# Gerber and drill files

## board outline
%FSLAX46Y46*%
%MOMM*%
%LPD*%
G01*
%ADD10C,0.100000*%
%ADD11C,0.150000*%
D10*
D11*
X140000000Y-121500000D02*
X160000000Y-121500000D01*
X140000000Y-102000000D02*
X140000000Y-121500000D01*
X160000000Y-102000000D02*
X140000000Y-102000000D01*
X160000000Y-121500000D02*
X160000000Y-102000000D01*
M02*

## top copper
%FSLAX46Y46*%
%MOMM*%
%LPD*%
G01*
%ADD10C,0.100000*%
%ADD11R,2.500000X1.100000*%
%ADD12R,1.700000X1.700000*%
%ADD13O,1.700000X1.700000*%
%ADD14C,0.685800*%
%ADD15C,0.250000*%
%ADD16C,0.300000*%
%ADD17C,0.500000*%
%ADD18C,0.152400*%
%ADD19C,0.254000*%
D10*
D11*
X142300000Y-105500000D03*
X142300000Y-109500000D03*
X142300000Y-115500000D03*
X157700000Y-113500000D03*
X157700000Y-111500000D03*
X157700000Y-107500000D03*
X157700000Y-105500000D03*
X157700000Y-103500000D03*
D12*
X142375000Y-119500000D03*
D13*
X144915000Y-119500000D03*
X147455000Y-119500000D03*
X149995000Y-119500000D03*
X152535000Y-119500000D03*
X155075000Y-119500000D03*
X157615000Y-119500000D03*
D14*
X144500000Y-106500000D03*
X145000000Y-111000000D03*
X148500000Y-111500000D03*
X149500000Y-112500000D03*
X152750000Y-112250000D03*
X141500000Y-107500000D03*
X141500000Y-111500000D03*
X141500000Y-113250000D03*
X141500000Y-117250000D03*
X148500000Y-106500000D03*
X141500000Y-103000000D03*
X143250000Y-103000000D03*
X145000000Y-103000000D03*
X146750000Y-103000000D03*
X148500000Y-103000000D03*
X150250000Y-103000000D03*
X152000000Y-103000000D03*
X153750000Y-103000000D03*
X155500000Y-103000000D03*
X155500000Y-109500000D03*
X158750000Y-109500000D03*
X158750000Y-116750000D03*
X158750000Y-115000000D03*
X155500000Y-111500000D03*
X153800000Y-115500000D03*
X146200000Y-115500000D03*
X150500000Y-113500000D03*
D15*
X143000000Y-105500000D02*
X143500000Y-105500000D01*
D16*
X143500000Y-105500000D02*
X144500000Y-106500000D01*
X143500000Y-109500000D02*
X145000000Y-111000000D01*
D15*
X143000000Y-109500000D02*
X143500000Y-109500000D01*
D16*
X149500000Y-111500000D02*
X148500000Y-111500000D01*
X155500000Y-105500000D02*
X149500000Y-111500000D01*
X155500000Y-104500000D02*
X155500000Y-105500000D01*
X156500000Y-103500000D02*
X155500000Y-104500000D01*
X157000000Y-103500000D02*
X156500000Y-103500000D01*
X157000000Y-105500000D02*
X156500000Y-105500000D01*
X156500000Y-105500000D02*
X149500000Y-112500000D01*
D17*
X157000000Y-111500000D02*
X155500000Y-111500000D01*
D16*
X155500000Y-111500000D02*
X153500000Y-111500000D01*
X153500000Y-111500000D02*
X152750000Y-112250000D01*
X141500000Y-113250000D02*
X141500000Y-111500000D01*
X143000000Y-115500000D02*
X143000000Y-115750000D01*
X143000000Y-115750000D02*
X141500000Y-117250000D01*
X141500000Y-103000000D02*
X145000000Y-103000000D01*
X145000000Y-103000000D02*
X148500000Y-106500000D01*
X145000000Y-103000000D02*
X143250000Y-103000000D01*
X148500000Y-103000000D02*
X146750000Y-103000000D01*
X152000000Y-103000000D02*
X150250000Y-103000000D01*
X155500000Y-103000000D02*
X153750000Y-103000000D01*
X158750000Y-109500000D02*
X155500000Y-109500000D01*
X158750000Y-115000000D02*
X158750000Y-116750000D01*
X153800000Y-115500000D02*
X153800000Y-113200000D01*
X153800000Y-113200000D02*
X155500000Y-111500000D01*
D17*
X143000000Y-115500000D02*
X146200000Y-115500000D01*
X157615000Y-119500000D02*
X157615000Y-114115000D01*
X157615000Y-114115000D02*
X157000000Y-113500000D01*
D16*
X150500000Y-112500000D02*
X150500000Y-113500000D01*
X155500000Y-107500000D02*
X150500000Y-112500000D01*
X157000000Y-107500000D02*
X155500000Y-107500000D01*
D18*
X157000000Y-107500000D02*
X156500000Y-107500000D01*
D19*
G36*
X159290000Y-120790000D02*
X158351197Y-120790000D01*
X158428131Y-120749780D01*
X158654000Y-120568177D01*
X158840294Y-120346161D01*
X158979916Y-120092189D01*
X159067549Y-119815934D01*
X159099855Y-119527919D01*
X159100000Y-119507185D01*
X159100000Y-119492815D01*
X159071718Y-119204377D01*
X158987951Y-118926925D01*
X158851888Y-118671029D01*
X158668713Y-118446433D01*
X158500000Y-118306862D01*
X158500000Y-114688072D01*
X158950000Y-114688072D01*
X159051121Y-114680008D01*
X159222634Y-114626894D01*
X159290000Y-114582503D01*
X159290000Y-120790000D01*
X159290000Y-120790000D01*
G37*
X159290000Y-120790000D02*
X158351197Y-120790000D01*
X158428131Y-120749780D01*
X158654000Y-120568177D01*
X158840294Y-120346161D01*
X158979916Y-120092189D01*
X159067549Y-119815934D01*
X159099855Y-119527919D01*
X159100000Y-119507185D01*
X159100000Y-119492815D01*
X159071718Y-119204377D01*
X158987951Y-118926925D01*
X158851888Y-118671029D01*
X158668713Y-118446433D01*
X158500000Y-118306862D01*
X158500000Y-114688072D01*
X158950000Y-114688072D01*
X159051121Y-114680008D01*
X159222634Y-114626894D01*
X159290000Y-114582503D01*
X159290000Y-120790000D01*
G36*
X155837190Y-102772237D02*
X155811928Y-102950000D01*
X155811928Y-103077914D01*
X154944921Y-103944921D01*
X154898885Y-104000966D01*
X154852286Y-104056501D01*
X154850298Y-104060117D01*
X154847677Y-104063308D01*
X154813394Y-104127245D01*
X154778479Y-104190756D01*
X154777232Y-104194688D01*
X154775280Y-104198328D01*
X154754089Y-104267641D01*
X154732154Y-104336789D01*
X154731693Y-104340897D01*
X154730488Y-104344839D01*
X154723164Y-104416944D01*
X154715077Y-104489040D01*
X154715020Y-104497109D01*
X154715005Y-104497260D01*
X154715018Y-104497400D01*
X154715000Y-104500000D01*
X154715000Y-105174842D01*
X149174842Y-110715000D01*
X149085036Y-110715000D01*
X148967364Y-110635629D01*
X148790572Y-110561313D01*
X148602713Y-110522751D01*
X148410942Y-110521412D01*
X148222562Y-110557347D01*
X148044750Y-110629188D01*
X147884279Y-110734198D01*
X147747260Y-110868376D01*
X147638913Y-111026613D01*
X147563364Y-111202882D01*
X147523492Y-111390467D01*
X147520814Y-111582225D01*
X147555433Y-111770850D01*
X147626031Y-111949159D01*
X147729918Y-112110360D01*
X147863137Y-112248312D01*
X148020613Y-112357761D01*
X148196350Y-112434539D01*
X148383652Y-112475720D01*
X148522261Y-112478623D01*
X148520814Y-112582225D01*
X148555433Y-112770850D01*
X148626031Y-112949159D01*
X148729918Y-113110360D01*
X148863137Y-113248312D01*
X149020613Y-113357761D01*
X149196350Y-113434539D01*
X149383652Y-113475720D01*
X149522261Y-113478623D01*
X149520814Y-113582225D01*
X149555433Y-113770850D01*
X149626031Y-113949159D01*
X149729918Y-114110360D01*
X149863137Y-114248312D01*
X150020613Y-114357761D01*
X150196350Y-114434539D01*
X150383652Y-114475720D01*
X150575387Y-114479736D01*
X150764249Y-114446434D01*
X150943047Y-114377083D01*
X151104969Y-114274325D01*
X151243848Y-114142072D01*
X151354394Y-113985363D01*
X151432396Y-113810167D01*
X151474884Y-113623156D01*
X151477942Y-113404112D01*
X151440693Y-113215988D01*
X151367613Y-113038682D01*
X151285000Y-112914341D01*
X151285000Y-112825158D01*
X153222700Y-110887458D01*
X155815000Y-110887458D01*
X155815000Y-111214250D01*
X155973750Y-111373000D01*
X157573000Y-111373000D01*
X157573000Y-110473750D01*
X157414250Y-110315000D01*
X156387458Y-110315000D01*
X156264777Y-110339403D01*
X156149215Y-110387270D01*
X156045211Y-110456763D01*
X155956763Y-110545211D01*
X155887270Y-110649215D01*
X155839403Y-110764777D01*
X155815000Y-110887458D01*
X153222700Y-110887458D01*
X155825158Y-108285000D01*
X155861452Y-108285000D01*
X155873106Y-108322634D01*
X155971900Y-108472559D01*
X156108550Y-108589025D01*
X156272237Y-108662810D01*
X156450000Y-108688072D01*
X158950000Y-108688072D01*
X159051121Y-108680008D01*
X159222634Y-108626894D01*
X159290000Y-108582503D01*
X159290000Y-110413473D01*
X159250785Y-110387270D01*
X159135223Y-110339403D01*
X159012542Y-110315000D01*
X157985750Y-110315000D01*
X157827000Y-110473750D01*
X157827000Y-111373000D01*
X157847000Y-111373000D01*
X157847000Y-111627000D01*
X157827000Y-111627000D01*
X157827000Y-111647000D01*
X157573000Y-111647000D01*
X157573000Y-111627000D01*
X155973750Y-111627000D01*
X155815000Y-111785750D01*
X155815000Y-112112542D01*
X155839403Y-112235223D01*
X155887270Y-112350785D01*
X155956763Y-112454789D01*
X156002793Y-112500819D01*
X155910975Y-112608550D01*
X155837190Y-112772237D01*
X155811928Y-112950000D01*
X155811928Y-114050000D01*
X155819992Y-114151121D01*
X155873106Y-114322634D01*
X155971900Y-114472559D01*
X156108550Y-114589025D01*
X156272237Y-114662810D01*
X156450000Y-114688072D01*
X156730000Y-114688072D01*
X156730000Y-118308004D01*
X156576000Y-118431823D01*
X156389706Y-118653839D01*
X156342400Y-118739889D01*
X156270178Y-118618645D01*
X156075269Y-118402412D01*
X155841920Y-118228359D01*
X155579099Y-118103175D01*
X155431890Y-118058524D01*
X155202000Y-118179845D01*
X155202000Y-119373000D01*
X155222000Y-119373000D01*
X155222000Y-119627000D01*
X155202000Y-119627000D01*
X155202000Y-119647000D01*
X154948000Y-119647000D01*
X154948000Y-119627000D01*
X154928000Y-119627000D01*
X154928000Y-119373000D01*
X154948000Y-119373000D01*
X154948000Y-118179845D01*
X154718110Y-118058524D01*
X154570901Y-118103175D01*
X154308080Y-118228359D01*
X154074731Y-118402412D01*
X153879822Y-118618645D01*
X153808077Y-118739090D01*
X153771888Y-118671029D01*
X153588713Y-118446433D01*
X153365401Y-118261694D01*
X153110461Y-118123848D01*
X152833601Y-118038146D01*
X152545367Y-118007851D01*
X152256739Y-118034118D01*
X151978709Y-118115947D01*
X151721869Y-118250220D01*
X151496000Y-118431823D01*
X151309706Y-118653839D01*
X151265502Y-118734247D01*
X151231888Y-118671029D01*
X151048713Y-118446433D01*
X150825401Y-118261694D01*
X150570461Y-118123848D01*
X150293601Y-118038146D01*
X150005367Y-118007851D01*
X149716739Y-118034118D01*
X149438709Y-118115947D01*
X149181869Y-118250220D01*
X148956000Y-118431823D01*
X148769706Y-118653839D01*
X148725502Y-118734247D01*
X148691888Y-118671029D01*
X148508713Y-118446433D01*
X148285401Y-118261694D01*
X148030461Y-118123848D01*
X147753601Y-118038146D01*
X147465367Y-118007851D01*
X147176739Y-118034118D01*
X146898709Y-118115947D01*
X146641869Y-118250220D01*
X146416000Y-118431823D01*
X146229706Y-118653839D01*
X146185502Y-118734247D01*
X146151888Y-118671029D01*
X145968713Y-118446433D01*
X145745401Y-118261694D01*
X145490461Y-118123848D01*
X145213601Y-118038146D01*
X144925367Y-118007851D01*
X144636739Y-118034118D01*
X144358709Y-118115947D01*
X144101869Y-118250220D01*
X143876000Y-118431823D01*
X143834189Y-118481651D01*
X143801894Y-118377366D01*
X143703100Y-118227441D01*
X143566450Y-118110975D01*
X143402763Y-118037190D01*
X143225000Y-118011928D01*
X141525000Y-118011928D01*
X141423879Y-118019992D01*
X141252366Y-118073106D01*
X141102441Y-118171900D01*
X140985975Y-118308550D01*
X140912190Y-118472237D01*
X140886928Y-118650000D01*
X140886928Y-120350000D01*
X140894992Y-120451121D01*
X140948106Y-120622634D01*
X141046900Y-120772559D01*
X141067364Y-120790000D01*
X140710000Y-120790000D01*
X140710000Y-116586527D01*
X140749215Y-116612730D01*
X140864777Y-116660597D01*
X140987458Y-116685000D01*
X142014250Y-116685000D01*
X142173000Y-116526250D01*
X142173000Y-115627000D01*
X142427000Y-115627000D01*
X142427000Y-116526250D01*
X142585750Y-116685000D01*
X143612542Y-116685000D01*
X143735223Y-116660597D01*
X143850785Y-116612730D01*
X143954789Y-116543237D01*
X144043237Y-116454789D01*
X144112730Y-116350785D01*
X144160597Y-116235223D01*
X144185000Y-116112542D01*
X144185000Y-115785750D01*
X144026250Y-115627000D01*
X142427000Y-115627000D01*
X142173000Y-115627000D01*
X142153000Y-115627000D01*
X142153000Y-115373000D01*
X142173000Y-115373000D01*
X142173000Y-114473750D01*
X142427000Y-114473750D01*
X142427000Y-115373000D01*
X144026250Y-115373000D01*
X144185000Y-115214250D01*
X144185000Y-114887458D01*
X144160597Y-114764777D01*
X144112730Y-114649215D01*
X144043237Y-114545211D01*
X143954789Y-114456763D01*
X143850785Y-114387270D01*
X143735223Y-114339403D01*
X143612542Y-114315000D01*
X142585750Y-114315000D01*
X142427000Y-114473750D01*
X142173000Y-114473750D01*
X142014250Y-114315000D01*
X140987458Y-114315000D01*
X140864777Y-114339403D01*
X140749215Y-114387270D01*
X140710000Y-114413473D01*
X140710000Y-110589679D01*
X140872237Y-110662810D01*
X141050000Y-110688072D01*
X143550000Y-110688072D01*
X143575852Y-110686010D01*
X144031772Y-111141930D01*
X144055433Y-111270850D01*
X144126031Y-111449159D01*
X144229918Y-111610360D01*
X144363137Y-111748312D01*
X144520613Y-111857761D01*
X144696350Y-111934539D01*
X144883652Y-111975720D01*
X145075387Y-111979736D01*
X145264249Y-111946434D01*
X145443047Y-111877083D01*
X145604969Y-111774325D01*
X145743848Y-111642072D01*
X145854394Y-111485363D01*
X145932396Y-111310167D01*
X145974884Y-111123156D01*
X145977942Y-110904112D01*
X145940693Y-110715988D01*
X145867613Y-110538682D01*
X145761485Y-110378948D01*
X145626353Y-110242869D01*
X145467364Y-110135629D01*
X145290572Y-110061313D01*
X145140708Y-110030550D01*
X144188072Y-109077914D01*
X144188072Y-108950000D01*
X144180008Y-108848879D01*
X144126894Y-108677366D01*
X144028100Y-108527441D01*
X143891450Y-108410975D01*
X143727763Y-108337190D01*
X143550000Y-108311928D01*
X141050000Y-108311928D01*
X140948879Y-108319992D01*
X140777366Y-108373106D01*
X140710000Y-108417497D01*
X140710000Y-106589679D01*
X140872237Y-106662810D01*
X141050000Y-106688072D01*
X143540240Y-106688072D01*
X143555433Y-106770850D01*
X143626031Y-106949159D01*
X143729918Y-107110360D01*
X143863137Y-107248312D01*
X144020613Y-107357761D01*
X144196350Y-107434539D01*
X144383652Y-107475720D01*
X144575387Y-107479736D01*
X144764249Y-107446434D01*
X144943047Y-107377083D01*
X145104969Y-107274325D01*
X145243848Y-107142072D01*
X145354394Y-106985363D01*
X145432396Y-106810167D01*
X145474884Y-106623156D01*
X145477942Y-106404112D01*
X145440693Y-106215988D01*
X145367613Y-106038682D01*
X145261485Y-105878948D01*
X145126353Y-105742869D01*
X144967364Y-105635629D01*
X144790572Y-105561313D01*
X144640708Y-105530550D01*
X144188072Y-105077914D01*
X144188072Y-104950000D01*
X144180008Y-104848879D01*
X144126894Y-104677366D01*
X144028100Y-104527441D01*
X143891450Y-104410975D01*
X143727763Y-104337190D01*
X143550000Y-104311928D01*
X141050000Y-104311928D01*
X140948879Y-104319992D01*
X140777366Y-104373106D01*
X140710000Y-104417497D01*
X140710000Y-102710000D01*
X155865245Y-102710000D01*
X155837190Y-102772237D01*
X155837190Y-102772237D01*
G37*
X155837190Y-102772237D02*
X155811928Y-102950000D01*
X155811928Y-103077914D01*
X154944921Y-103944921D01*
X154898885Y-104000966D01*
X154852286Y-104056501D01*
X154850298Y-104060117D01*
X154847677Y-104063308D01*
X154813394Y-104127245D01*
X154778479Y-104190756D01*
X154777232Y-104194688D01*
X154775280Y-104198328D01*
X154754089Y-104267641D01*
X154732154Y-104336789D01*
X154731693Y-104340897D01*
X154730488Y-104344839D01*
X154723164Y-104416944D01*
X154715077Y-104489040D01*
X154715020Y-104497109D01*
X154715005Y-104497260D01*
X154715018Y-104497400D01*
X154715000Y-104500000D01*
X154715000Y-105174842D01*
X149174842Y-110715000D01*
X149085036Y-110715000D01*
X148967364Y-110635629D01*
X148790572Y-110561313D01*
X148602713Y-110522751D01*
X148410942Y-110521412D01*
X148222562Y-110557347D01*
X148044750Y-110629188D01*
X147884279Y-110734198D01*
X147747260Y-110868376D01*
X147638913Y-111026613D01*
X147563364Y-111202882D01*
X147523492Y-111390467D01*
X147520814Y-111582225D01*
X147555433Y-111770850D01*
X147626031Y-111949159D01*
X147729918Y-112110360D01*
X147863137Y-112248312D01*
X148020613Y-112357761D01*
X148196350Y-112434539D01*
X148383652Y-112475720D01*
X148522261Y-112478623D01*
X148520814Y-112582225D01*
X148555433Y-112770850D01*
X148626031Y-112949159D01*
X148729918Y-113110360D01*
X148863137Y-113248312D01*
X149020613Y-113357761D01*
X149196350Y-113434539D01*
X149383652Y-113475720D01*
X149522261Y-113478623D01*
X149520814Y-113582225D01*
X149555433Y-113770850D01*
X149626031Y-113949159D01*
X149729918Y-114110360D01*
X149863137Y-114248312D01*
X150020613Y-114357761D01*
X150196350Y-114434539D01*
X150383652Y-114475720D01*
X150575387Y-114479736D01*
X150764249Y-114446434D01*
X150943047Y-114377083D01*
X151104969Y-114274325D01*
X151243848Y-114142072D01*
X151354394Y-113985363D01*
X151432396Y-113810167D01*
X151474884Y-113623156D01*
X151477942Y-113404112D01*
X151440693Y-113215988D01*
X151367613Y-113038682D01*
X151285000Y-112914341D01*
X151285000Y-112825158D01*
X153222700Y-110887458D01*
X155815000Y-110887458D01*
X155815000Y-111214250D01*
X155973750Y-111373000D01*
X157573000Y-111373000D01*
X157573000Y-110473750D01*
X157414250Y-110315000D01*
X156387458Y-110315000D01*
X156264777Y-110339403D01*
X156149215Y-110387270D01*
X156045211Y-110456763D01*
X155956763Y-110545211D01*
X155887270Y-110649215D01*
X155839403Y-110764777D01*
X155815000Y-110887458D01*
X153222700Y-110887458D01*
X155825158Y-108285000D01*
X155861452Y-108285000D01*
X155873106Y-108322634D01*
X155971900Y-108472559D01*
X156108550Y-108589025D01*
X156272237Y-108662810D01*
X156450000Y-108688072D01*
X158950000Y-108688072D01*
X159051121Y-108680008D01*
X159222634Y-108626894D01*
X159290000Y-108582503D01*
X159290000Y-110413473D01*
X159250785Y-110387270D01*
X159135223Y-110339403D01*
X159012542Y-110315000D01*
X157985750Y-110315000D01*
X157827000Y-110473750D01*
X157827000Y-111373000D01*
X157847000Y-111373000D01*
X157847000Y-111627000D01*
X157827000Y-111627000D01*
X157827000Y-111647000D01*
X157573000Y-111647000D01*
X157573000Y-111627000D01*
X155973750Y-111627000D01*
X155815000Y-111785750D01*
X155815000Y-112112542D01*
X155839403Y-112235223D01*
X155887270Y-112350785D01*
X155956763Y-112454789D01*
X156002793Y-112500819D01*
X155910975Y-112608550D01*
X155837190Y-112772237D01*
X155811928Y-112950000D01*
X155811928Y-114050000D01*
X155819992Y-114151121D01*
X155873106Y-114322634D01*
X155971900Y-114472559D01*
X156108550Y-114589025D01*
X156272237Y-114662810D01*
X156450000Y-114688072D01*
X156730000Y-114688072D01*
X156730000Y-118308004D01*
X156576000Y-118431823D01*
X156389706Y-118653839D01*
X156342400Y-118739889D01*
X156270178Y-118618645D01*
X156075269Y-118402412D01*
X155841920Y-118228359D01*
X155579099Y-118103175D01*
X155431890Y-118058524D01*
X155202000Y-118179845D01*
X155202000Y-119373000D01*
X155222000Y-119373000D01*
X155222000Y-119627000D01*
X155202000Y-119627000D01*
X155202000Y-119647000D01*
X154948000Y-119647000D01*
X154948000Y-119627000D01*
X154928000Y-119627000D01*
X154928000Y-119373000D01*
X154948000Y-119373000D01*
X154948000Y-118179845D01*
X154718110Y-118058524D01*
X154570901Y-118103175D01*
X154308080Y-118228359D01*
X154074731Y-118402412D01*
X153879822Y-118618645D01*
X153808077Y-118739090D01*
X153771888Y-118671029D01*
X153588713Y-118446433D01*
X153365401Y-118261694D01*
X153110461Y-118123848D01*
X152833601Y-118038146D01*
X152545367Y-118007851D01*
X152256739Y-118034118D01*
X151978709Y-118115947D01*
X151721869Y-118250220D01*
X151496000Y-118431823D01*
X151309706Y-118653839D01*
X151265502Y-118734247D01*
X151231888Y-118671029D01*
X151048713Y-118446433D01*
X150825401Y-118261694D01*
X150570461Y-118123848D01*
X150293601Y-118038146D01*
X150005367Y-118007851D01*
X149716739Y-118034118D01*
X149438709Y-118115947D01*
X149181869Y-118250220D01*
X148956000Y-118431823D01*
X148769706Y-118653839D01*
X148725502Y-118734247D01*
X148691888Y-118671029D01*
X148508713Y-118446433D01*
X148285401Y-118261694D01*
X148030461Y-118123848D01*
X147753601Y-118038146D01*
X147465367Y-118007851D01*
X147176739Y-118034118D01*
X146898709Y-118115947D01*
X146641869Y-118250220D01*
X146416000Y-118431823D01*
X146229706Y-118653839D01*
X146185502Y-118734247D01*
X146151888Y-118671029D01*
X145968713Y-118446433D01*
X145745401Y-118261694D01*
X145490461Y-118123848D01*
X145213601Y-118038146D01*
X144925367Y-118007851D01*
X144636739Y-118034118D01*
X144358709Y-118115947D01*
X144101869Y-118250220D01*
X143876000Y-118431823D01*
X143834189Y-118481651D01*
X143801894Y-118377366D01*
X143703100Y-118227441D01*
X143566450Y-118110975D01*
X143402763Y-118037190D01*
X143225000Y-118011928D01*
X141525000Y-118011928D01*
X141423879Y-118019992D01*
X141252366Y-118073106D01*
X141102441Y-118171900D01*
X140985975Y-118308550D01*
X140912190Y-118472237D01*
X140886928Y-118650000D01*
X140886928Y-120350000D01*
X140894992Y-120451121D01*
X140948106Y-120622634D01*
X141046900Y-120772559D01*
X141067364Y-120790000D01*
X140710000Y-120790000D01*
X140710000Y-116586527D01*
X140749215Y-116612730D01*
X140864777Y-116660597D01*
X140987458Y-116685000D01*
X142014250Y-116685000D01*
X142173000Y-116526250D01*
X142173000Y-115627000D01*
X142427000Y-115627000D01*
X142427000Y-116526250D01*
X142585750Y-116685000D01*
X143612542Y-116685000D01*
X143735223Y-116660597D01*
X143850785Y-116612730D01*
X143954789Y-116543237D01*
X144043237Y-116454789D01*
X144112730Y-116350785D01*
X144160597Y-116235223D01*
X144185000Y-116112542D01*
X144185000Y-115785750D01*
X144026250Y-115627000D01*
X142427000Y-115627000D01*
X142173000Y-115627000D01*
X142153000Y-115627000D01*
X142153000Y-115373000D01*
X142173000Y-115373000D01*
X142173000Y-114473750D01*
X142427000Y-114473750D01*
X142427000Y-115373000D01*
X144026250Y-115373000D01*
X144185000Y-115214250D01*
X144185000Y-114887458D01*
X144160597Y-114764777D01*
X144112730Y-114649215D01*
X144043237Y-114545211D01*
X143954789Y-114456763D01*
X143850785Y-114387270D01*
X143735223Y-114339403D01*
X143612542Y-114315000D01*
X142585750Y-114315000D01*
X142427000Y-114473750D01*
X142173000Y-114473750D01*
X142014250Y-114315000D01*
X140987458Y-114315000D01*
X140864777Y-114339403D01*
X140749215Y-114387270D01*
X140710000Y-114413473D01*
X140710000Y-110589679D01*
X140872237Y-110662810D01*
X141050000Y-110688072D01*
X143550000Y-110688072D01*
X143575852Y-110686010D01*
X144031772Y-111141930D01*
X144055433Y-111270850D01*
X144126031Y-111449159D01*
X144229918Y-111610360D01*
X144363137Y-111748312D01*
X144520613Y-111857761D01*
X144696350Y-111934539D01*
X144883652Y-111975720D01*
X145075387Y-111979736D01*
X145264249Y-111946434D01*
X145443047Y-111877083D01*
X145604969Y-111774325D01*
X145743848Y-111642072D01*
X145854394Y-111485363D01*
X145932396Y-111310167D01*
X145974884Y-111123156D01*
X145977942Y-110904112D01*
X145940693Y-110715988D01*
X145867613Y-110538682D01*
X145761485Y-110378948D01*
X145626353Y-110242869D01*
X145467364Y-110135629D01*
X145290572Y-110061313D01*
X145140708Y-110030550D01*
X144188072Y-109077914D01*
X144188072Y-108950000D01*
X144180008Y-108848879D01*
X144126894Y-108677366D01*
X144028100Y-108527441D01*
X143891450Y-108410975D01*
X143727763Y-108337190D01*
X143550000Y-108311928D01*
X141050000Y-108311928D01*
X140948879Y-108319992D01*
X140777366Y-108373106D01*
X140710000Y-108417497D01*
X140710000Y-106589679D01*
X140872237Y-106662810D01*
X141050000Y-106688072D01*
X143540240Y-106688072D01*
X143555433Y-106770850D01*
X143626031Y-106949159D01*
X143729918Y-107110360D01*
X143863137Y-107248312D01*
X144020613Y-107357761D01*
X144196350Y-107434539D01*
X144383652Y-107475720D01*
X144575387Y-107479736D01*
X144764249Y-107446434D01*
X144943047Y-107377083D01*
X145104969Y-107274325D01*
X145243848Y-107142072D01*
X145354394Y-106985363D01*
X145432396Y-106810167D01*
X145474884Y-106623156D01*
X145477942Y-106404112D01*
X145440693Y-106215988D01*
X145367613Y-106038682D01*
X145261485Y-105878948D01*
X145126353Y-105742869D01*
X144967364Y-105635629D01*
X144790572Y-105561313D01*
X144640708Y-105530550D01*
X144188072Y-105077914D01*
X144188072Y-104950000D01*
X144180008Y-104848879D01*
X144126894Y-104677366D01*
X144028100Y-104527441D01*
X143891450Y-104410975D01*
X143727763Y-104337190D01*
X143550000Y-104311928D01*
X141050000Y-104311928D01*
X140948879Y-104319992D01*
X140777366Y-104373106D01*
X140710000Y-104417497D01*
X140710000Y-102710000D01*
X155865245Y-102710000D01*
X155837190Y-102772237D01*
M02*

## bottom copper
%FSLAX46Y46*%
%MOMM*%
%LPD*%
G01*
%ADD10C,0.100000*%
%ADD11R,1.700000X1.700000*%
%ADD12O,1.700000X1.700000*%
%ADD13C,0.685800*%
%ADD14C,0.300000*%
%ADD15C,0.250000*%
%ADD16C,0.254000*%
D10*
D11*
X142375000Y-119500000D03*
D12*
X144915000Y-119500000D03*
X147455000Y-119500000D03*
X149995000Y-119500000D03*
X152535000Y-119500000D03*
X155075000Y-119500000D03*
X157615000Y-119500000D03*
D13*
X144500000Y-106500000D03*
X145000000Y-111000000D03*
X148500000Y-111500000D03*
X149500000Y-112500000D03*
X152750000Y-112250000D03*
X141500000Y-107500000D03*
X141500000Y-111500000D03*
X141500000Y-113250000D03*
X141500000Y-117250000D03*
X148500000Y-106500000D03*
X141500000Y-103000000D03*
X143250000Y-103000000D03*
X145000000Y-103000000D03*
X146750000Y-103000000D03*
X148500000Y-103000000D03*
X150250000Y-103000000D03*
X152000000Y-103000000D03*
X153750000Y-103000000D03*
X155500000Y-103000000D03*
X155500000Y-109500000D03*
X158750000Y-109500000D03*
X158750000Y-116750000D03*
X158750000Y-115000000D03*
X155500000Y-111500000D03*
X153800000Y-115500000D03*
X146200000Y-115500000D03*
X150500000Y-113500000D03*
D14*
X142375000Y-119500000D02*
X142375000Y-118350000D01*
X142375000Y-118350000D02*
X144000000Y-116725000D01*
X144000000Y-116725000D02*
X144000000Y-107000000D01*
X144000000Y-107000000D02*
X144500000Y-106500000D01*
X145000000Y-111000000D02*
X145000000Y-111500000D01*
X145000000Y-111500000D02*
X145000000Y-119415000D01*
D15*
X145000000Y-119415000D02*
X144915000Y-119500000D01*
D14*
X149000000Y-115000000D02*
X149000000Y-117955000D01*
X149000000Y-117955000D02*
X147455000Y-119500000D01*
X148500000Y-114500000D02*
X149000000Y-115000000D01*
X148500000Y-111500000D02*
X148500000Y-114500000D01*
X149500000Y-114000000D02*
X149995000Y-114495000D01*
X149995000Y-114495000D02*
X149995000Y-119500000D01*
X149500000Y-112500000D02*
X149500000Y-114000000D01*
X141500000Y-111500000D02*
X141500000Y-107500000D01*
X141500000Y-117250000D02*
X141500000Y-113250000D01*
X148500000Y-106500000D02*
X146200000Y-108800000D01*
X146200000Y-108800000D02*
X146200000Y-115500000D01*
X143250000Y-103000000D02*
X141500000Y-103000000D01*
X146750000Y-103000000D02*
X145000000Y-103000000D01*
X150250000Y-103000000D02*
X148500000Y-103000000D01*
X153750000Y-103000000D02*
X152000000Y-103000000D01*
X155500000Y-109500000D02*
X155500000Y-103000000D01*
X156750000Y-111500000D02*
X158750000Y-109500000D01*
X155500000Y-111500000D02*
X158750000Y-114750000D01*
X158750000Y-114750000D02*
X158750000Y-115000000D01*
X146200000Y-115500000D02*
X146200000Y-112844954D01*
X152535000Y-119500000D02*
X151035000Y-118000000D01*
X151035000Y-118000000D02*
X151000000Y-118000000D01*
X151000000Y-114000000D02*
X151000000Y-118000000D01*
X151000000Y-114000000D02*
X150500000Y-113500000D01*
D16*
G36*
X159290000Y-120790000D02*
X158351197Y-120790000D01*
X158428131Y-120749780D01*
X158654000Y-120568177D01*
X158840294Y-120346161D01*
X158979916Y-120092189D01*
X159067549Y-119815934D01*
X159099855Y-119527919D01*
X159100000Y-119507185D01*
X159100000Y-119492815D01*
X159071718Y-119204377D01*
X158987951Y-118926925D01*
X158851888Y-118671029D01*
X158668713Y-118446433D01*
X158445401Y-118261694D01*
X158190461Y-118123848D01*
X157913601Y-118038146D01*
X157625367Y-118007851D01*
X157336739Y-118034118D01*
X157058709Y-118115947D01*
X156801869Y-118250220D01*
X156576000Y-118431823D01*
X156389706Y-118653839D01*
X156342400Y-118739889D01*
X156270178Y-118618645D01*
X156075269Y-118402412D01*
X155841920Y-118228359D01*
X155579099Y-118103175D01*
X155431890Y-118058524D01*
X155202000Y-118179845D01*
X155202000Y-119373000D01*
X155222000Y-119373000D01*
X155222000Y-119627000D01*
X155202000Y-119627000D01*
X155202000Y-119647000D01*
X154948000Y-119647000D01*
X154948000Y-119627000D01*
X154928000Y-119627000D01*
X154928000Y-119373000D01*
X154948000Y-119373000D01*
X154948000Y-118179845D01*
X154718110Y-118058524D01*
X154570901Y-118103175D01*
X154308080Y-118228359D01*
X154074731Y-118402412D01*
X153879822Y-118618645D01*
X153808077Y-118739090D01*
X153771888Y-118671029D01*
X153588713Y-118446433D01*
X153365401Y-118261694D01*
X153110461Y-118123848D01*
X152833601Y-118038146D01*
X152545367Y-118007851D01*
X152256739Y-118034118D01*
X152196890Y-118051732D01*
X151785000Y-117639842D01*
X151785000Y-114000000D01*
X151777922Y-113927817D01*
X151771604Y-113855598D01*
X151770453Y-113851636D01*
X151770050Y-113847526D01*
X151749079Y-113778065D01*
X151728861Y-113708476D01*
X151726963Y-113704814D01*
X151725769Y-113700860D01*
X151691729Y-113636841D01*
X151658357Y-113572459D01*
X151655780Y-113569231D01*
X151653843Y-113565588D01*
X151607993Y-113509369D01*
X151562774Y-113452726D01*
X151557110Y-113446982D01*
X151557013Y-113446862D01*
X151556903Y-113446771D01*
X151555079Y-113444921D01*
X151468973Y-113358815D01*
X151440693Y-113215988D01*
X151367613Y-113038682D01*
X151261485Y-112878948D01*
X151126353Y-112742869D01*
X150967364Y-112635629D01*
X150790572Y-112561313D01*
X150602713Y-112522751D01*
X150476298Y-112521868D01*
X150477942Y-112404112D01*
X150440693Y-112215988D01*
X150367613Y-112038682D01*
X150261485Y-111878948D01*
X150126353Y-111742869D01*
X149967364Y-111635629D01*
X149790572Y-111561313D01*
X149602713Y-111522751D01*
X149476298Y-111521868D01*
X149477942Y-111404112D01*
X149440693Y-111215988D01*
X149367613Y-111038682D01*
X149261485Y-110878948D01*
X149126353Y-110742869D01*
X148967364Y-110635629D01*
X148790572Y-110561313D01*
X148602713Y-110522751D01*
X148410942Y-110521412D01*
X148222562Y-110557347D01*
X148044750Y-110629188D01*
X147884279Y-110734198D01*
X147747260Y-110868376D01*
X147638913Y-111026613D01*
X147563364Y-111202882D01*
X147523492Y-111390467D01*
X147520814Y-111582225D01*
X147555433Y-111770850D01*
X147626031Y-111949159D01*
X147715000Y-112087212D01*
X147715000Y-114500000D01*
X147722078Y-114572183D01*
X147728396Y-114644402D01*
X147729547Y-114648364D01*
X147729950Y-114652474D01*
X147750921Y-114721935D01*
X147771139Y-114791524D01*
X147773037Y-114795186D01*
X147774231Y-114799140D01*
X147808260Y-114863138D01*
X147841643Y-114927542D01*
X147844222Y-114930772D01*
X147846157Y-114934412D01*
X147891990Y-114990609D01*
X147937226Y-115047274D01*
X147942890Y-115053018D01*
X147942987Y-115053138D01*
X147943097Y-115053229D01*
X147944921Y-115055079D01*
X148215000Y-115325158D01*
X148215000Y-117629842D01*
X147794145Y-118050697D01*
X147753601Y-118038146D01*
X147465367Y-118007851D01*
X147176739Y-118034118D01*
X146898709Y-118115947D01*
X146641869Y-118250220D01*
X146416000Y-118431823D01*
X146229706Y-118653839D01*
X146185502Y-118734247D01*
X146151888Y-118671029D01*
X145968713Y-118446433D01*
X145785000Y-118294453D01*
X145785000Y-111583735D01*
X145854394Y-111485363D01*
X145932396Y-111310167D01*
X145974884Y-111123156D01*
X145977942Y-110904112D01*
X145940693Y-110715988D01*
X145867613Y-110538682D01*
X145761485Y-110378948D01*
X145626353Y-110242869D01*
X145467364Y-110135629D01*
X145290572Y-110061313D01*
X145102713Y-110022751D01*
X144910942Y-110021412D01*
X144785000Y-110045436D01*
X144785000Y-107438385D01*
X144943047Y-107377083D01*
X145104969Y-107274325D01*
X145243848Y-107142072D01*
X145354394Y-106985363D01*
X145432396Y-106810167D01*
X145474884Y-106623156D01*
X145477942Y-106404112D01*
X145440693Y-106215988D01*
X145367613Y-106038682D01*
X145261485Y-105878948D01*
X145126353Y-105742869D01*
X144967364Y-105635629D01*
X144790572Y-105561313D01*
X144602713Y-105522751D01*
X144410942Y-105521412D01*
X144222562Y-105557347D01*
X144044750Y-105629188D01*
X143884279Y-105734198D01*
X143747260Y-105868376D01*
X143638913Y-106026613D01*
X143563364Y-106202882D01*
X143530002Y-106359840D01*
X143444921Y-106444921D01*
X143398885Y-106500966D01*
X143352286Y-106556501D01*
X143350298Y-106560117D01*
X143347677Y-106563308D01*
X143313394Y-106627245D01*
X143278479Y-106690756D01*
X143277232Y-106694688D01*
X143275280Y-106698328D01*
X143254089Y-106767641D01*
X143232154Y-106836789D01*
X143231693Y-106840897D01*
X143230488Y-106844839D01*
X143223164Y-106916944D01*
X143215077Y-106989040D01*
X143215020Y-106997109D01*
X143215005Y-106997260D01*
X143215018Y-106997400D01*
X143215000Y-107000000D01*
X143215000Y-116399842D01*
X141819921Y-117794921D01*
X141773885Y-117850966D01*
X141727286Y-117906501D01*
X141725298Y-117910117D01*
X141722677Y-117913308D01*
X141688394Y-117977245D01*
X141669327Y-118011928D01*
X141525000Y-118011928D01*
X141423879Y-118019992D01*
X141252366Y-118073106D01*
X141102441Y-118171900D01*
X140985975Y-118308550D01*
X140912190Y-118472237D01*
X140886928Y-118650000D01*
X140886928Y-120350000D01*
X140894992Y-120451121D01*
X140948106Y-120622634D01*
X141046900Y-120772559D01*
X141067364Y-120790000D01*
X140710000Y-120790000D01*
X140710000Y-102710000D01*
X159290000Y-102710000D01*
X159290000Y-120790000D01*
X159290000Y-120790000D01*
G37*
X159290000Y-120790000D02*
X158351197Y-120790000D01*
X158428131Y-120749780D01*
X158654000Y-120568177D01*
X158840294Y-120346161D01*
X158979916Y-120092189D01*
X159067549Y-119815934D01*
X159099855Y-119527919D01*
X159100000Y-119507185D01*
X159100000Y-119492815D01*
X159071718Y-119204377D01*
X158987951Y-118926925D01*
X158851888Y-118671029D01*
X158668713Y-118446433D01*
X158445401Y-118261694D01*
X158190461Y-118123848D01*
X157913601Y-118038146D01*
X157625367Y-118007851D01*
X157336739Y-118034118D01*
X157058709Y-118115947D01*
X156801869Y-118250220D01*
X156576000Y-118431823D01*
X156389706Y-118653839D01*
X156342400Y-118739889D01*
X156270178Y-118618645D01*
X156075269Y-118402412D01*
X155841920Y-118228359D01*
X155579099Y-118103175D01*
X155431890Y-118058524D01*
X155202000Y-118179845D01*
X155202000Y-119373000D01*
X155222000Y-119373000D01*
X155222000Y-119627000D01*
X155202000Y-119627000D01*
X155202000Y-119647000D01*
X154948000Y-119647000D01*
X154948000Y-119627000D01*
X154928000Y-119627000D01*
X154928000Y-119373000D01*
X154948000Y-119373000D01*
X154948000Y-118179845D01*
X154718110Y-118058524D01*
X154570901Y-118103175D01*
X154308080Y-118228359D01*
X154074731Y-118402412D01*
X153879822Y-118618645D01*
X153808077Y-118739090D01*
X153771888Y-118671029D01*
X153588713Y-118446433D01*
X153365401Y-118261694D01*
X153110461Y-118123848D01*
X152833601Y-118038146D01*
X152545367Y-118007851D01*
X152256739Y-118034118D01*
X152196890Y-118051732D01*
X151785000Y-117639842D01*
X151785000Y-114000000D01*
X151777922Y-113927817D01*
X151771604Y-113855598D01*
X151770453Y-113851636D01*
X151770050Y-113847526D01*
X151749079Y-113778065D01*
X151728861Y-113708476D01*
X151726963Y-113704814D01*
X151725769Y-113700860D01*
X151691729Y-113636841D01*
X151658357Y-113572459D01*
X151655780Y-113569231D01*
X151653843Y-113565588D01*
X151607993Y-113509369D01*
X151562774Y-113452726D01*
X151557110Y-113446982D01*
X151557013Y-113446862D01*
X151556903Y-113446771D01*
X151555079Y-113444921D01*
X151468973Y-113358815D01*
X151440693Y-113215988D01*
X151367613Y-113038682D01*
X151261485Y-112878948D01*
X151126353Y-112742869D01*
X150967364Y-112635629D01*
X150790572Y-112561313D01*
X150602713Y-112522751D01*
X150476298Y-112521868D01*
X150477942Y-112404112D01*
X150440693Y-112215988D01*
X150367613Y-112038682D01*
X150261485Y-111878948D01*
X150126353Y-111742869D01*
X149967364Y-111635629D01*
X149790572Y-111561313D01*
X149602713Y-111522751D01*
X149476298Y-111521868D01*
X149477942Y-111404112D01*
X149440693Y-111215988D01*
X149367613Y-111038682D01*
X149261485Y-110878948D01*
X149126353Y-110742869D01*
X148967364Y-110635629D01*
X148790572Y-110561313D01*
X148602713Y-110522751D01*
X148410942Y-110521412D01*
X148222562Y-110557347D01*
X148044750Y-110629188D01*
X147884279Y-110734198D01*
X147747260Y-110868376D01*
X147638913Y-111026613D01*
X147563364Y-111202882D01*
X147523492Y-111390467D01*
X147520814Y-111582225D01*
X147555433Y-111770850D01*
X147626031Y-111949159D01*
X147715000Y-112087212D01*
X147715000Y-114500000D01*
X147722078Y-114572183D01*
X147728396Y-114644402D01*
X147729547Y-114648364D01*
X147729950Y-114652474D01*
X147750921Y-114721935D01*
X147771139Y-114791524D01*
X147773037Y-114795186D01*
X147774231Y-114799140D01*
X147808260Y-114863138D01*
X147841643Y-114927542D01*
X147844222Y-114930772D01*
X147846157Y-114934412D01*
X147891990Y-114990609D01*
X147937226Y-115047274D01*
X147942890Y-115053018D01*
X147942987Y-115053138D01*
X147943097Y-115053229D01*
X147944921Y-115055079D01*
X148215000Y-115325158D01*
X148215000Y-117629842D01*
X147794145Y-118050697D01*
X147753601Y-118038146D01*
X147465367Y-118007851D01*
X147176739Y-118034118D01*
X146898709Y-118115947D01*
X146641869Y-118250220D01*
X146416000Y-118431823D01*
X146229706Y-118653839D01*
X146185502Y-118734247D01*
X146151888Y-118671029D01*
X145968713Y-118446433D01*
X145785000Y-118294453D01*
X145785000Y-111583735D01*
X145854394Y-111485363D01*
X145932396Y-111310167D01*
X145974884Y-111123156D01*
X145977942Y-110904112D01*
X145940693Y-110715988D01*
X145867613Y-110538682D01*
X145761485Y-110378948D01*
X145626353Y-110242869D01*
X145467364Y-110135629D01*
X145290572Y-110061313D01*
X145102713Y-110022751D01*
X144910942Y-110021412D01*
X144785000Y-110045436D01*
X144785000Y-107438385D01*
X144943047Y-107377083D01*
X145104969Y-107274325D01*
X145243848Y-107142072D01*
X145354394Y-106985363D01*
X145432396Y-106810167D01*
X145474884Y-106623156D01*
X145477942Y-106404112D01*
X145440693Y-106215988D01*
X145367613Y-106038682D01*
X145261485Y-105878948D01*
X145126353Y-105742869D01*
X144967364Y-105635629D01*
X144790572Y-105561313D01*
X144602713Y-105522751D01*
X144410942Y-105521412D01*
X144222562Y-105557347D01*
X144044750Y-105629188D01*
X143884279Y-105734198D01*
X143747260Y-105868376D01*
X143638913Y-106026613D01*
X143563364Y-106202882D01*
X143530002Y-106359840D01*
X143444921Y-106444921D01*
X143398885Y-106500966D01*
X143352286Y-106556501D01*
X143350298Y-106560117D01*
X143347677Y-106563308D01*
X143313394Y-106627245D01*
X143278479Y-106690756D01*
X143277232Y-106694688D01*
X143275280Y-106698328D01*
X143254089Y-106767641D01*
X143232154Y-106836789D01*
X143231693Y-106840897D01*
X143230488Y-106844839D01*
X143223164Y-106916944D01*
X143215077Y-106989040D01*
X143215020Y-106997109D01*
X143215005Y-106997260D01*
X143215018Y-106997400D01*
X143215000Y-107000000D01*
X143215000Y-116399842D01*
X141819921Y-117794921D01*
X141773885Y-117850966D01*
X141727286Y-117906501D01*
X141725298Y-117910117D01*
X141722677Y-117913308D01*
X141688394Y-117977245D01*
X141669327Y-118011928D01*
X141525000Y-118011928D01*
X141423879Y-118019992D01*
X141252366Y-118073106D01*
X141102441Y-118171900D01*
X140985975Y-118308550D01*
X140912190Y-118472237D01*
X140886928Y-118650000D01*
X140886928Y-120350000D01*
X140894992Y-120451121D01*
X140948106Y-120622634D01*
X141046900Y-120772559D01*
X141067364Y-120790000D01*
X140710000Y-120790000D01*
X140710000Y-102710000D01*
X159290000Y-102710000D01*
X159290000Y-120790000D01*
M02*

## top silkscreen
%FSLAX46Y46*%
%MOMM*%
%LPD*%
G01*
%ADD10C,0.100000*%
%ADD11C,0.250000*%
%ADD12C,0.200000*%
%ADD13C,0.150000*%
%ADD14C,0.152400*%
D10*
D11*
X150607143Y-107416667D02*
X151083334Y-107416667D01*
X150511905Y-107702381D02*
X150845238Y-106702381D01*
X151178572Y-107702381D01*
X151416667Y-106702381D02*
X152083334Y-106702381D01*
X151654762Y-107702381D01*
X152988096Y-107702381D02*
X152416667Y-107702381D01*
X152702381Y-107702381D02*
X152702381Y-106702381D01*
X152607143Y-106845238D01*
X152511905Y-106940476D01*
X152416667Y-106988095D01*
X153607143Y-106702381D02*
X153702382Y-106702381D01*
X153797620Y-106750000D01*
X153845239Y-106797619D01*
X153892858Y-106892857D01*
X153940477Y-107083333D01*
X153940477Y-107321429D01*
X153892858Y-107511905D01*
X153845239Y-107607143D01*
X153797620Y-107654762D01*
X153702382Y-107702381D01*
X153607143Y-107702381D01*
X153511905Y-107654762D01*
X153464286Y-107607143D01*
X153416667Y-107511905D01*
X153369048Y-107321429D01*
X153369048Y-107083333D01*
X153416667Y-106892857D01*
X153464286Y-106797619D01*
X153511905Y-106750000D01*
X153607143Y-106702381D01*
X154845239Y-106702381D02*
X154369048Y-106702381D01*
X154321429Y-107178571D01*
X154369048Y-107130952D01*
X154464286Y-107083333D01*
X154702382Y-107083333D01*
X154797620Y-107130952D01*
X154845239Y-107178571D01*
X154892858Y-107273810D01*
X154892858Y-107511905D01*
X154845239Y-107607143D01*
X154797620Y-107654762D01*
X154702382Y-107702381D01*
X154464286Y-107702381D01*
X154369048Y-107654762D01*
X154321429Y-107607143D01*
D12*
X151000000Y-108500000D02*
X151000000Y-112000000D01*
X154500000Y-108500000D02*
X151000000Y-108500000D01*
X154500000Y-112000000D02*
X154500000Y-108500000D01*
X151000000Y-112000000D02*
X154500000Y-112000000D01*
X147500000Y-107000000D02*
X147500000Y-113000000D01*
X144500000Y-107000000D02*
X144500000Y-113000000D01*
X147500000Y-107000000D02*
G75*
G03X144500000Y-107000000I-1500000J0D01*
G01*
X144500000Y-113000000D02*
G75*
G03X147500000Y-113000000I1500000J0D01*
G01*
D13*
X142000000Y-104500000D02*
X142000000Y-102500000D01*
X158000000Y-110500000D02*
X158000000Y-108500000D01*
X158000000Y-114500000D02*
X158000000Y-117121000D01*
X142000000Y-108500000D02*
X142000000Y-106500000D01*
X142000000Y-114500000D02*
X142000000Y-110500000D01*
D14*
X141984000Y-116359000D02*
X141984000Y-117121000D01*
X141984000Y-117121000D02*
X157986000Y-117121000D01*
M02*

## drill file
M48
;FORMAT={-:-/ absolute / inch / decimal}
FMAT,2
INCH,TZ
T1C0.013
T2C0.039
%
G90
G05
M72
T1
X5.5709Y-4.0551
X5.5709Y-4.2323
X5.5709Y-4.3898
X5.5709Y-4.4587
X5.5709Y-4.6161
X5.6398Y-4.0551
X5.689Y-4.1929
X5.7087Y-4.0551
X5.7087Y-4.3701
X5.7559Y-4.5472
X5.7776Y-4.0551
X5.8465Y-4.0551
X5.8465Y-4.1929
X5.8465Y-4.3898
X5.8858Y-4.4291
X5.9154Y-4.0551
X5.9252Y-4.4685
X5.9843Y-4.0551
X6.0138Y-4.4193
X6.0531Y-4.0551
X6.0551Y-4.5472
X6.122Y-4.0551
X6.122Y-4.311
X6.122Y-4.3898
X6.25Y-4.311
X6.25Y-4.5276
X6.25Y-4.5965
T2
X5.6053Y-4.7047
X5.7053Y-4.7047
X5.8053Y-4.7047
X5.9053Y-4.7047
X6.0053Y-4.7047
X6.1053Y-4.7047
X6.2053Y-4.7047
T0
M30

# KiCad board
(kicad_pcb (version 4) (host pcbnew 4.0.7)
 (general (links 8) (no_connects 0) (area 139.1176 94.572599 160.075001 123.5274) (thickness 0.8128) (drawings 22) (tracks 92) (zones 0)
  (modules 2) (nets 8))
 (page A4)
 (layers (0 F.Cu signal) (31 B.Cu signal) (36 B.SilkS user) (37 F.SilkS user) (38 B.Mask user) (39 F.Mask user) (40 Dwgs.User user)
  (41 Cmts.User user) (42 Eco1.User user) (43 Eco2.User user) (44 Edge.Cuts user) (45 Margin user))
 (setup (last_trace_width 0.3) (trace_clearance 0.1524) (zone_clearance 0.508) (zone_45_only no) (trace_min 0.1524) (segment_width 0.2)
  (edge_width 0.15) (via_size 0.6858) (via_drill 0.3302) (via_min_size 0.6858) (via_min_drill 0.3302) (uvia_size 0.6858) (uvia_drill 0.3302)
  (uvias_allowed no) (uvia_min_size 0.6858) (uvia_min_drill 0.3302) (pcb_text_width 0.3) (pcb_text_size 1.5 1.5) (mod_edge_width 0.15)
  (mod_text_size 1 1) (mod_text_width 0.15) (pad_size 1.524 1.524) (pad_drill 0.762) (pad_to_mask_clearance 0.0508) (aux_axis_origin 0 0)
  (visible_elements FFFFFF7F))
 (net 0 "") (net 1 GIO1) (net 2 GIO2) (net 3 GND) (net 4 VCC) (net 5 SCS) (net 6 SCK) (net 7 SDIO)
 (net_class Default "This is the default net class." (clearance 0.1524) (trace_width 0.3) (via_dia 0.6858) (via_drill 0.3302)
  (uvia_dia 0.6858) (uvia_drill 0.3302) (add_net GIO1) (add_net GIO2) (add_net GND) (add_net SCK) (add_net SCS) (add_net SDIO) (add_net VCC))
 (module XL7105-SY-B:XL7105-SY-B (layer F.Cu) (at 143 103.5)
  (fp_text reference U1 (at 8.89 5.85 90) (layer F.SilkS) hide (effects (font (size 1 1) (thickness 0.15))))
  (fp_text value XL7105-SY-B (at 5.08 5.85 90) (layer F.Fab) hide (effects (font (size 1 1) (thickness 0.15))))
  (fp_line (start -1 1) (end -1 -1) (layer F.SilkS) (width 0.15))
  (fp_line (start 15 7) (end 15 5) (layer F.SilkS) (width 0.15))
  (fp_line (start 15 11) (end 15 13.621) (layer F.SilkS) (width 0.15))
  (fp_line (start -1 5) (end -1 3) (layer F.SilkS) (width 0.15))
  (fp_line (start -1 11) (end -1 7) (layer F.SilkS) (width 0.15))
  (fp_line (start -1.016 12.859) (end -1.016 13.621) (layer F.SilkS) (width 0.1524))
  (fp_line (start -1.016 13.621) (end 14.986 13.621) (layer F.SilkS) (width 0.1524))
  (pad 2 smd rect (at 0 2) (size 2.5 1.1) (drill (offset -0.7 0)) (layers F.Cu F.Mask) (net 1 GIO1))
  (pad 4 smd rect (at 0 6) (size 2.5 1.1) (drill (offset -0.7 0)) (layers F.Cu F.Mask) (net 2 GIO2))
  (pad 7 smd rect (at 0 12) (size 2.5 1.1) (drill (offset -0.7 0)) (layers F.Cu F.Mask) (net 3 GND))
  (pad 9 smd rect (at 14 10) (size 2.5 1.1) (drill (offset 0.7 0)) (layers F.Cu F.Mask) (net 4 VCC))
  (pad 10 smd rect (at 14 8) (size 2.5 1.1) (drill (offset 0.7 0)) (layers F.Cu F.Mask) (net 3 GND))
  (pad 12 smd rect (at 14 4) (size 2.5 1.1) (drill (offset 0.7 0)) (layers F.Cu F.Mask) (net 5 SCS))
  (pad 13 smd rect (at 14 2) (size 2.5 1.1) (drill (offset 0.7 0)) (layers F.Cu F.Mask) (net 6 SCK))
  (pad 14 smd rect (at 14 0) (size 2.5 1.1) (drill (offset 0.7 0)) (layers F.Cu F.Mask) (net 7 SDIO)))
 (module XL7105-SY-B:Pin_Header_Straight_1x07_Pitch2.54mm (layer F.Cu) (at 142.375 119.5 90)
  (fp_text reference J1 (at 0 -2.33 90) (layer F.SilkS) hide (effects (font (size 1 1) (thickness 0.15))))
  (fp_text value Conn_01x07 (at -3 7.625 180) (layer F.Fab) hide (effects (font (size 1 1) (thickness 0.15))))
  (pad 1 thru_hole rect (at 0 0 90) (size 1.7 1.7) (drill 1) (layers *.Cu *.Mask) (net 1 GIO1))
  (pad 2 thru_hole oval (at 0 2.54 90) (size 1.7 1.7) (drill 1) (layers *.Cu *.Mask) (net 2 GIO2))
  (pad 3 thru_hole oval (at 0 5.08 90) (size 1.7 1.7) (drill 1) (layers *.Cu *.Mask) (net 7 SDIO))
  (pad 4 thru_hole oval (at 0 7.62 90) (size 1.7 1.7) (drill 1) (layers *.Cu *.Mask) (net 6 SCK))
  (pad 5 thru_hole oval (at 0 10.16 90) (size 1.7 1.7) (drill 1) (layers *.Cu *.Mask) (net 5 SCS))
  (pad 6 thru_hole oval (at 0 12.7 90) (size 1.7 1.7) (drill 1) (layers *.Cu *.Mask) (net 3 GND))
  (pad 7 thru_hole oval (at 0 15.24 90) (size 1.7 1.7) (drill 1) (layers *.Cu *.Mask) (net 4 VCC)))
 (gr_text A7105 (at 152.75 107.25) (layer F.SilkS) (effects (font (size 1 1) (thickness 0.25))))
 (gr_line (start 151 108.5) (end 151 112) (layer F.SilkS) (width 0.2))
 (gr_line (start 154.5 108.5) (end 151 108.5) (layer F.SilkS) (width 0.2))
 (gr_line (start 154.5 112) (end 154.5 108.5) (layer F.SilkS) (width 0.2))
 (gr_line (start 151 112) (end 154.5 112) (layer F.SilkS) (width 0.2))
 (gr_line (start 147.5 107) (end 147.5 113) (layer F.SilkS) (width 0.2))
 (gr_line (start 144.5 107) (end 144.5 113) (layer F.SilkS) (width 0.2))
 (gr_arc (start 146 107) (end 144.5 107) (angle 180) (layer F.SilkS) (width 0.2))
 (gr_arc (start 146 113) (end 147.5 113) (angle 180) (layer F.SilkS) (width 0.2))
 (gr_line (start 140 121.5) (end 160 121.5) (layer Edge.Cuts) (width 0.15))
 (gr_line (start 140 102) (end 140 121.5) (layer Edge.Cuts) (width 0.15))
 (gr_line (start 160 102) (end 140 102) (layer Edge.Cuts) (width 0.15))
 (gr_line (start 160 121.5) (end 160 102) (layer Edge.Cuts) (width 0.15))
 (segment (start 142.375 119.5) (end 142.375 118.35) (width 0.3) (layer B.Cu) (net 1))
 (segment (start 142.375 118.35) (end 144 116.725) (width 0.3) (layer B.Cu) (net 1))
 (segment (start 144 116.725) (end 144 107) (width 0.3) (layer B.Cu) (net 1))
 (segment (start 144 107) (end 144.5 106.5) (width 0.3) (layer B.Cu) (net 1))
 (segment (start 143 105.5) (end 143.5 105.5) (width 0.25) (layer F.Cu) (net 1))
 (via (at 144.5 106.5) (size 0.6858) (drill 0.3302) (layers F.Cu B.Cu) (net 1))
 (segment (start 143.5 105.5) (end 144.5 106.5) (width 0.3) (layer F.Cu) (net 1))
 (segment (start 145 111) (end 145 111.5) (width 0.3) (layer B.Cu) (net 2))
 (segment (start 143.5 109.5) (end 145 111) (width 0.3) (layer F.Cu) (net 2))
 (via (at 145 111) (size 0.6858) (drill 0.3302) (layers F.Cu B.Cu) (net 2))
 (segment (start 143 109.5) (end 143.5 109.5) (width 0.25) (layer F.Cu) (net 2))
 (segment (start 145 111.5) (end 145 119.415) (width 0.3) (layer B.Cu) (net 2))
 (segment (start 145 119.415) (end 144.915 119.5) (width 0.25) (layer B.Cu) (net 2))
 (segment (start 149 115) (end 149 117.955) (width 0.3) (layer B.Cu) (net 7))
 (segment (start 149 117.955) (end 147.455 119.5) (width 0.3) (layer B.Cu) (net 7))
 (segment (start 148.5 114.5) (end 149 115) (width 0.3) (layer B.Cu) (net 7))
 (segment (start 148.5 111.5) (end 148.5 114.5) (width 0.3) (layer B.Cu) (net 7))
 (segment (start 149.5 111.5) (end 148.5 111.5) (width 0.3) (layer F.Cu) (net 7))
 (segment (start 155.5 105.5) (end 149.5 111.5) (width 0.3) (layer F.Cu) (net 7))
 (segment (start 155.5 104.5) (end 155.5 105.5) (width 0.3) (layer F.Cu) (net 7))
 (segment (start 156.5 103.5) (end 155.5 104.5) (width 0.3) (layer F.Cu) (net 7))
 (segment (start 157 103.5) (end 156.5 103.5) (width 0.3) (layer F.Cu) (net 7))
 (via (at 148.5 111.5) (size 0.6858) (drill 0.3302) (layers F.Cu B.Cu) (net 7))
 (segment (start 149.5 114) (end 149.995 114.495) (width 0.3) (layer B.Cu) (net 6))
 (segment (start 149.995 114.495) (end 149.995 119.5) (width 0.3) (layer B.Cu) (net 6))
 (segment (start 149.5 112.5) (end 149.5 114) (width 0.3) (layer B.Cu) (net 6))
 (segment (start 157 105.5) (end 156.5 105.5) (width 0.3) (layer F.Cu) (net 6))
 (segment (start 156.5 105.5) (end 149.5 112.5) (width 0.3) (layer F.Cu) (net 6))
 (via (at 149.5 112.5) (size 0.6858) (drill 0.3302) (layers F.Cu B.Cu) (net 6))
 (segment (start 157 111.5) (end 155.5 111.5) (width 0.5) (layer F.Cu) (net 3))
 (segment (start 155.5 111.5) (end 153.5 111.5) (width 0.3) (layer F.Cu) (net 3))
 (segment (start 153.5 111.5) (end 152.75 112.25) (width 0.3) (layer F.Cu) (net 3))
 (via (at 152.75 112.25) (size 0.6858) (drill 0.3302) (layers F.Cu B.Cu) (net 3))
 (segment (start 141.5 111.5) (end 141.5 107.5) (width 0.3) (layer B.Cu) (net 3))
 (via (at 141.5 107.5) (size 0.6858) (drill 0.3302) (layers F.Cu B.Cu) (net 3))
 (segment (start 141.5 113.25) (end 141.5 111.5) (width 0.3) (layer F.Cu) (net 3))
 (via (at 141.5 111.5) (size 0.6858) (drill 0.3302) (layers F.Cu B.Cu) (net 3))
 (segment (start 141.5 117.25) (end 141.5 113.25) (width 0.3) (layer B.Cu) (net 3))
 (via (at 141.5 113.25) (size 0.6858) (drill 0.3302) (layers F.Cu B.Cu) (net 3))
 (segment (start 143 115.5) (end 143 115.75) (width 0.3) (layer F.Cu) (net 3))
 (segment (start 143 115.75) (end 141.5 117.25) (width 0.3) (layer F.Cu) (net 3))
 (via (at 141.5 117.25) (size 0.6858) (drill 0.3302) (layers F.Cu B.Cu) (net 3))
 (segment (start 148.5 106.5) (end 146.2 108.8) (width 0.3) (layer B.Cu) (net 3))
 (segment (start 146.2 108.8) (end 146.2 115.5) (width 0.3) (layer B.Cu) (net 3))
 (segment (start 141.5 103) (end 145 103) (width 0.3) (layer F.Cu) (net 3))
 (segment (start 145 103) (end 148.5 106.5) (width 0.3) (layer F.Cu) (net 3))
 (via (at 148.5 106.5) (size 0.6858) (drill 0.3302) (layers F.Cu B.Cu) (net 3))
 (segment (start 143.25 103) (end 141.5 103) (width 0.3) (layer B.Cu) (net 3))
 (via (at 141.5 103) (size 0.6858) (drill 0.3302) (layers F.Cu B.Cu) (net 3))
 (segment (start 145 103) (end 143.25 103) (width 0.3) (layer F.Cu) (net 3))
 (via (at 143.25 103) (size 0.6858) (drill 0.3302) (layers F.Cu B.Cu) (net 3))
 (segment (start 146.75 103) (end 145 103) (width 0.3) (layer B.Cu) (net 3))
 (via (at 145 103) (size 0.6858) (drill 0.3302) (layers F.Cu B.Cu) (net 3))
 (segment (start 148.5 103) (end 146.75 103) (width 0.3) (layer F.Cu) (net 3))
 (via (at 146.75 103) (size 0.6858) (drill 0.3302) (layers F.Cu B.Cu) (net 3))
 (segment (start 150.25 103) (end 148.5 103) (width 0.3) (layer B.Cu) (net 3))
 (via (at 148.5 103) (size 0.6858) (drill 0.3302) (layers F.Cu B.Cu) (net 3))
 (segment (start 152 103) (end 150.25 103) (width 0.3) (layer F.Cu) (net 3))
 (via (at 150.25 103) (size 0.6858) (drill 0.3302) (layers F.Cu B.Cu) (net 3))
 (segment (start 153.75 103) (end 152 103) (width 0.3) (layer B.Cu) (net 3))
 (via (at 152 103) (size 0.6858) (drill 0.3302) (layers F.Cu B.Cu) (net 3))
 (segment (start 155.5 103) (end 153.75 103) (width 0.3) (layer F.Cu) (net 3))
 (via (at 153.75 103) (size 0.6858) (drill 0.3302) (layers F.Cu B.Cu) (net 3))
 (segment (start 155.5 109.5) (end 155.5 103) (width 0.3) (layer B.Cu) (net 3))
 (via (at 155.5 103) (size 0.6858) (drill 0.3302) (layers F.Cu B.Cu) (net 3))
 (via (at 155.5 109.5) (size 0.6858) (drill 0.3302) (layers F.Cu B.Cu) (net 3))
 (segment (start 158.75 109.5) (end 155.5 109.5) (width 0.3) (layer F.Cu) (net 3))
 (segment (start 156.75 111.5) (end 158.75 109.5) (width 0.3) (layer B.Cu) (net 3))
 (via (at 158.75 109.5) (size 0.6858) (drill 0.3302) (layers F.Cu B.Cu) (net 3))
 (segment (start 158.75 115) (end 158.75 116.75) (width 0.3) (layer F.Cu) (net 3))
 (via (at 158.75 116.75) (size 0.6858) (drill 0.3302) (layers F.Cu B.Cu) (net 3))
 (segment (start 155.5 111.5) (end 158.75 114.75) (width 0.3) (layer B.Cu) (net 3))
 (segment (start 158.75 114.75) (end 158.75 115) (width 0.3) (layer B.Cu) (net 3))
 (via (at 158.75 115) (size 0.6858) (drill 0.3302) (layers F.Cu B.Cu) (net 3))
 (segment (start 153.8 115.5) (end 153.8 113.2) (width 0.3) (layer F.Cu) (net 3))
 (segment (start 153.8 113.2) (end 155.5 111.5) (width 0.3) (layer F.Cu) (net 3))
 (via (at 155.5 111.5) (size 0.6858) (drill 0.3302) (layers F.Cu B.Cu) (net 3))
 (segment (start 146.2 115.5) (end 146.2 112.844954) (width 0.3) (layer B.Cu) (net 3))
 (via (at 153.8 115.5) (size 0.6858) (drill 0.3302) (layers F.Cu B.Cu) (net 3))
 (segment (start 143 115.5) (end 146.2 115.5) (width 0.5) (layer F.Cu) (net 3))
 (via (at 146.2 115.5) (size 0.6858) (drill 0.3302) (layers F.Cu B.Cu) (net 3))
 (segment (start 157.615 119.5) (end 157.615 114.115) (width 0.5) (layer F.Cu) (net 4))
 (segment (start 157.615 114.115) (end 157 113.5) (width 0.5) (layer F.Cu) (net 4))
 (segment (start 152.535 119.5) (end 151.035 118) (width 0.3) (layer B.Cu) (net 5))
 (segment (start 151.035 118) (end 151 118) (width 0.3) (layer B.Cu) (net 5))
 (segment (start 151 114) (end 151 118) (width 0.3) (layer B.Cu) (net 5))
 (segment (start 151 114) (end 150.5 113.5) (width 0.3) (layer B.Cu) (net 5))
 (segment (start 150.5 112.5) (end 150.5 113.5) (width 0.3) (layer F.Cu) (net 5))
 (segment (start 155.5 107.5) (end 150.5 112.5) (width 0.3) (layer F.Cu) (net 5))
 (segment (start 157 107.5) (end 155.5 107.5) (width 0.3) (layer F.Cu) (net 5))
 (segment (start 157 107.5) (end 156.5 107.5) (width 0.1524) (layer F.Cu) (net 5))
 (via (at 150.5 113.5) (size 0.6858) (drill 0.3302) (layers F.Cu B.Cu) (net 5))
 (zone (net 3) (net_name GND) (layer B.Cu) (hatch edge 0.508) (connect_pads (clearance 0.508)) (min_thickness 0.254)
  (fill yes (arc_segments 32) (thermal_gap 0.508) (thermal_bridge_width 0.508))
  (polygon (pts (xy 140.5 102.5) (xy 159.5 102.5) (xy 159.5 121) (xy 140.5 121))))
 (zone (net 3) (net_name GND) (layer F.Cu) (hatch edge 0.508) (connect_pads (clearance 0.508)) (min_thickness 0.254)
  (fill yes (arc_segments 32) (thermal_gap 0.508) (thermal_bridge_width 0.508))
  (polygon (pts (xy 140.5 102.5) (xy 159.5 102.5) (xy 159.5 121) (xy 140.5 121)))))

